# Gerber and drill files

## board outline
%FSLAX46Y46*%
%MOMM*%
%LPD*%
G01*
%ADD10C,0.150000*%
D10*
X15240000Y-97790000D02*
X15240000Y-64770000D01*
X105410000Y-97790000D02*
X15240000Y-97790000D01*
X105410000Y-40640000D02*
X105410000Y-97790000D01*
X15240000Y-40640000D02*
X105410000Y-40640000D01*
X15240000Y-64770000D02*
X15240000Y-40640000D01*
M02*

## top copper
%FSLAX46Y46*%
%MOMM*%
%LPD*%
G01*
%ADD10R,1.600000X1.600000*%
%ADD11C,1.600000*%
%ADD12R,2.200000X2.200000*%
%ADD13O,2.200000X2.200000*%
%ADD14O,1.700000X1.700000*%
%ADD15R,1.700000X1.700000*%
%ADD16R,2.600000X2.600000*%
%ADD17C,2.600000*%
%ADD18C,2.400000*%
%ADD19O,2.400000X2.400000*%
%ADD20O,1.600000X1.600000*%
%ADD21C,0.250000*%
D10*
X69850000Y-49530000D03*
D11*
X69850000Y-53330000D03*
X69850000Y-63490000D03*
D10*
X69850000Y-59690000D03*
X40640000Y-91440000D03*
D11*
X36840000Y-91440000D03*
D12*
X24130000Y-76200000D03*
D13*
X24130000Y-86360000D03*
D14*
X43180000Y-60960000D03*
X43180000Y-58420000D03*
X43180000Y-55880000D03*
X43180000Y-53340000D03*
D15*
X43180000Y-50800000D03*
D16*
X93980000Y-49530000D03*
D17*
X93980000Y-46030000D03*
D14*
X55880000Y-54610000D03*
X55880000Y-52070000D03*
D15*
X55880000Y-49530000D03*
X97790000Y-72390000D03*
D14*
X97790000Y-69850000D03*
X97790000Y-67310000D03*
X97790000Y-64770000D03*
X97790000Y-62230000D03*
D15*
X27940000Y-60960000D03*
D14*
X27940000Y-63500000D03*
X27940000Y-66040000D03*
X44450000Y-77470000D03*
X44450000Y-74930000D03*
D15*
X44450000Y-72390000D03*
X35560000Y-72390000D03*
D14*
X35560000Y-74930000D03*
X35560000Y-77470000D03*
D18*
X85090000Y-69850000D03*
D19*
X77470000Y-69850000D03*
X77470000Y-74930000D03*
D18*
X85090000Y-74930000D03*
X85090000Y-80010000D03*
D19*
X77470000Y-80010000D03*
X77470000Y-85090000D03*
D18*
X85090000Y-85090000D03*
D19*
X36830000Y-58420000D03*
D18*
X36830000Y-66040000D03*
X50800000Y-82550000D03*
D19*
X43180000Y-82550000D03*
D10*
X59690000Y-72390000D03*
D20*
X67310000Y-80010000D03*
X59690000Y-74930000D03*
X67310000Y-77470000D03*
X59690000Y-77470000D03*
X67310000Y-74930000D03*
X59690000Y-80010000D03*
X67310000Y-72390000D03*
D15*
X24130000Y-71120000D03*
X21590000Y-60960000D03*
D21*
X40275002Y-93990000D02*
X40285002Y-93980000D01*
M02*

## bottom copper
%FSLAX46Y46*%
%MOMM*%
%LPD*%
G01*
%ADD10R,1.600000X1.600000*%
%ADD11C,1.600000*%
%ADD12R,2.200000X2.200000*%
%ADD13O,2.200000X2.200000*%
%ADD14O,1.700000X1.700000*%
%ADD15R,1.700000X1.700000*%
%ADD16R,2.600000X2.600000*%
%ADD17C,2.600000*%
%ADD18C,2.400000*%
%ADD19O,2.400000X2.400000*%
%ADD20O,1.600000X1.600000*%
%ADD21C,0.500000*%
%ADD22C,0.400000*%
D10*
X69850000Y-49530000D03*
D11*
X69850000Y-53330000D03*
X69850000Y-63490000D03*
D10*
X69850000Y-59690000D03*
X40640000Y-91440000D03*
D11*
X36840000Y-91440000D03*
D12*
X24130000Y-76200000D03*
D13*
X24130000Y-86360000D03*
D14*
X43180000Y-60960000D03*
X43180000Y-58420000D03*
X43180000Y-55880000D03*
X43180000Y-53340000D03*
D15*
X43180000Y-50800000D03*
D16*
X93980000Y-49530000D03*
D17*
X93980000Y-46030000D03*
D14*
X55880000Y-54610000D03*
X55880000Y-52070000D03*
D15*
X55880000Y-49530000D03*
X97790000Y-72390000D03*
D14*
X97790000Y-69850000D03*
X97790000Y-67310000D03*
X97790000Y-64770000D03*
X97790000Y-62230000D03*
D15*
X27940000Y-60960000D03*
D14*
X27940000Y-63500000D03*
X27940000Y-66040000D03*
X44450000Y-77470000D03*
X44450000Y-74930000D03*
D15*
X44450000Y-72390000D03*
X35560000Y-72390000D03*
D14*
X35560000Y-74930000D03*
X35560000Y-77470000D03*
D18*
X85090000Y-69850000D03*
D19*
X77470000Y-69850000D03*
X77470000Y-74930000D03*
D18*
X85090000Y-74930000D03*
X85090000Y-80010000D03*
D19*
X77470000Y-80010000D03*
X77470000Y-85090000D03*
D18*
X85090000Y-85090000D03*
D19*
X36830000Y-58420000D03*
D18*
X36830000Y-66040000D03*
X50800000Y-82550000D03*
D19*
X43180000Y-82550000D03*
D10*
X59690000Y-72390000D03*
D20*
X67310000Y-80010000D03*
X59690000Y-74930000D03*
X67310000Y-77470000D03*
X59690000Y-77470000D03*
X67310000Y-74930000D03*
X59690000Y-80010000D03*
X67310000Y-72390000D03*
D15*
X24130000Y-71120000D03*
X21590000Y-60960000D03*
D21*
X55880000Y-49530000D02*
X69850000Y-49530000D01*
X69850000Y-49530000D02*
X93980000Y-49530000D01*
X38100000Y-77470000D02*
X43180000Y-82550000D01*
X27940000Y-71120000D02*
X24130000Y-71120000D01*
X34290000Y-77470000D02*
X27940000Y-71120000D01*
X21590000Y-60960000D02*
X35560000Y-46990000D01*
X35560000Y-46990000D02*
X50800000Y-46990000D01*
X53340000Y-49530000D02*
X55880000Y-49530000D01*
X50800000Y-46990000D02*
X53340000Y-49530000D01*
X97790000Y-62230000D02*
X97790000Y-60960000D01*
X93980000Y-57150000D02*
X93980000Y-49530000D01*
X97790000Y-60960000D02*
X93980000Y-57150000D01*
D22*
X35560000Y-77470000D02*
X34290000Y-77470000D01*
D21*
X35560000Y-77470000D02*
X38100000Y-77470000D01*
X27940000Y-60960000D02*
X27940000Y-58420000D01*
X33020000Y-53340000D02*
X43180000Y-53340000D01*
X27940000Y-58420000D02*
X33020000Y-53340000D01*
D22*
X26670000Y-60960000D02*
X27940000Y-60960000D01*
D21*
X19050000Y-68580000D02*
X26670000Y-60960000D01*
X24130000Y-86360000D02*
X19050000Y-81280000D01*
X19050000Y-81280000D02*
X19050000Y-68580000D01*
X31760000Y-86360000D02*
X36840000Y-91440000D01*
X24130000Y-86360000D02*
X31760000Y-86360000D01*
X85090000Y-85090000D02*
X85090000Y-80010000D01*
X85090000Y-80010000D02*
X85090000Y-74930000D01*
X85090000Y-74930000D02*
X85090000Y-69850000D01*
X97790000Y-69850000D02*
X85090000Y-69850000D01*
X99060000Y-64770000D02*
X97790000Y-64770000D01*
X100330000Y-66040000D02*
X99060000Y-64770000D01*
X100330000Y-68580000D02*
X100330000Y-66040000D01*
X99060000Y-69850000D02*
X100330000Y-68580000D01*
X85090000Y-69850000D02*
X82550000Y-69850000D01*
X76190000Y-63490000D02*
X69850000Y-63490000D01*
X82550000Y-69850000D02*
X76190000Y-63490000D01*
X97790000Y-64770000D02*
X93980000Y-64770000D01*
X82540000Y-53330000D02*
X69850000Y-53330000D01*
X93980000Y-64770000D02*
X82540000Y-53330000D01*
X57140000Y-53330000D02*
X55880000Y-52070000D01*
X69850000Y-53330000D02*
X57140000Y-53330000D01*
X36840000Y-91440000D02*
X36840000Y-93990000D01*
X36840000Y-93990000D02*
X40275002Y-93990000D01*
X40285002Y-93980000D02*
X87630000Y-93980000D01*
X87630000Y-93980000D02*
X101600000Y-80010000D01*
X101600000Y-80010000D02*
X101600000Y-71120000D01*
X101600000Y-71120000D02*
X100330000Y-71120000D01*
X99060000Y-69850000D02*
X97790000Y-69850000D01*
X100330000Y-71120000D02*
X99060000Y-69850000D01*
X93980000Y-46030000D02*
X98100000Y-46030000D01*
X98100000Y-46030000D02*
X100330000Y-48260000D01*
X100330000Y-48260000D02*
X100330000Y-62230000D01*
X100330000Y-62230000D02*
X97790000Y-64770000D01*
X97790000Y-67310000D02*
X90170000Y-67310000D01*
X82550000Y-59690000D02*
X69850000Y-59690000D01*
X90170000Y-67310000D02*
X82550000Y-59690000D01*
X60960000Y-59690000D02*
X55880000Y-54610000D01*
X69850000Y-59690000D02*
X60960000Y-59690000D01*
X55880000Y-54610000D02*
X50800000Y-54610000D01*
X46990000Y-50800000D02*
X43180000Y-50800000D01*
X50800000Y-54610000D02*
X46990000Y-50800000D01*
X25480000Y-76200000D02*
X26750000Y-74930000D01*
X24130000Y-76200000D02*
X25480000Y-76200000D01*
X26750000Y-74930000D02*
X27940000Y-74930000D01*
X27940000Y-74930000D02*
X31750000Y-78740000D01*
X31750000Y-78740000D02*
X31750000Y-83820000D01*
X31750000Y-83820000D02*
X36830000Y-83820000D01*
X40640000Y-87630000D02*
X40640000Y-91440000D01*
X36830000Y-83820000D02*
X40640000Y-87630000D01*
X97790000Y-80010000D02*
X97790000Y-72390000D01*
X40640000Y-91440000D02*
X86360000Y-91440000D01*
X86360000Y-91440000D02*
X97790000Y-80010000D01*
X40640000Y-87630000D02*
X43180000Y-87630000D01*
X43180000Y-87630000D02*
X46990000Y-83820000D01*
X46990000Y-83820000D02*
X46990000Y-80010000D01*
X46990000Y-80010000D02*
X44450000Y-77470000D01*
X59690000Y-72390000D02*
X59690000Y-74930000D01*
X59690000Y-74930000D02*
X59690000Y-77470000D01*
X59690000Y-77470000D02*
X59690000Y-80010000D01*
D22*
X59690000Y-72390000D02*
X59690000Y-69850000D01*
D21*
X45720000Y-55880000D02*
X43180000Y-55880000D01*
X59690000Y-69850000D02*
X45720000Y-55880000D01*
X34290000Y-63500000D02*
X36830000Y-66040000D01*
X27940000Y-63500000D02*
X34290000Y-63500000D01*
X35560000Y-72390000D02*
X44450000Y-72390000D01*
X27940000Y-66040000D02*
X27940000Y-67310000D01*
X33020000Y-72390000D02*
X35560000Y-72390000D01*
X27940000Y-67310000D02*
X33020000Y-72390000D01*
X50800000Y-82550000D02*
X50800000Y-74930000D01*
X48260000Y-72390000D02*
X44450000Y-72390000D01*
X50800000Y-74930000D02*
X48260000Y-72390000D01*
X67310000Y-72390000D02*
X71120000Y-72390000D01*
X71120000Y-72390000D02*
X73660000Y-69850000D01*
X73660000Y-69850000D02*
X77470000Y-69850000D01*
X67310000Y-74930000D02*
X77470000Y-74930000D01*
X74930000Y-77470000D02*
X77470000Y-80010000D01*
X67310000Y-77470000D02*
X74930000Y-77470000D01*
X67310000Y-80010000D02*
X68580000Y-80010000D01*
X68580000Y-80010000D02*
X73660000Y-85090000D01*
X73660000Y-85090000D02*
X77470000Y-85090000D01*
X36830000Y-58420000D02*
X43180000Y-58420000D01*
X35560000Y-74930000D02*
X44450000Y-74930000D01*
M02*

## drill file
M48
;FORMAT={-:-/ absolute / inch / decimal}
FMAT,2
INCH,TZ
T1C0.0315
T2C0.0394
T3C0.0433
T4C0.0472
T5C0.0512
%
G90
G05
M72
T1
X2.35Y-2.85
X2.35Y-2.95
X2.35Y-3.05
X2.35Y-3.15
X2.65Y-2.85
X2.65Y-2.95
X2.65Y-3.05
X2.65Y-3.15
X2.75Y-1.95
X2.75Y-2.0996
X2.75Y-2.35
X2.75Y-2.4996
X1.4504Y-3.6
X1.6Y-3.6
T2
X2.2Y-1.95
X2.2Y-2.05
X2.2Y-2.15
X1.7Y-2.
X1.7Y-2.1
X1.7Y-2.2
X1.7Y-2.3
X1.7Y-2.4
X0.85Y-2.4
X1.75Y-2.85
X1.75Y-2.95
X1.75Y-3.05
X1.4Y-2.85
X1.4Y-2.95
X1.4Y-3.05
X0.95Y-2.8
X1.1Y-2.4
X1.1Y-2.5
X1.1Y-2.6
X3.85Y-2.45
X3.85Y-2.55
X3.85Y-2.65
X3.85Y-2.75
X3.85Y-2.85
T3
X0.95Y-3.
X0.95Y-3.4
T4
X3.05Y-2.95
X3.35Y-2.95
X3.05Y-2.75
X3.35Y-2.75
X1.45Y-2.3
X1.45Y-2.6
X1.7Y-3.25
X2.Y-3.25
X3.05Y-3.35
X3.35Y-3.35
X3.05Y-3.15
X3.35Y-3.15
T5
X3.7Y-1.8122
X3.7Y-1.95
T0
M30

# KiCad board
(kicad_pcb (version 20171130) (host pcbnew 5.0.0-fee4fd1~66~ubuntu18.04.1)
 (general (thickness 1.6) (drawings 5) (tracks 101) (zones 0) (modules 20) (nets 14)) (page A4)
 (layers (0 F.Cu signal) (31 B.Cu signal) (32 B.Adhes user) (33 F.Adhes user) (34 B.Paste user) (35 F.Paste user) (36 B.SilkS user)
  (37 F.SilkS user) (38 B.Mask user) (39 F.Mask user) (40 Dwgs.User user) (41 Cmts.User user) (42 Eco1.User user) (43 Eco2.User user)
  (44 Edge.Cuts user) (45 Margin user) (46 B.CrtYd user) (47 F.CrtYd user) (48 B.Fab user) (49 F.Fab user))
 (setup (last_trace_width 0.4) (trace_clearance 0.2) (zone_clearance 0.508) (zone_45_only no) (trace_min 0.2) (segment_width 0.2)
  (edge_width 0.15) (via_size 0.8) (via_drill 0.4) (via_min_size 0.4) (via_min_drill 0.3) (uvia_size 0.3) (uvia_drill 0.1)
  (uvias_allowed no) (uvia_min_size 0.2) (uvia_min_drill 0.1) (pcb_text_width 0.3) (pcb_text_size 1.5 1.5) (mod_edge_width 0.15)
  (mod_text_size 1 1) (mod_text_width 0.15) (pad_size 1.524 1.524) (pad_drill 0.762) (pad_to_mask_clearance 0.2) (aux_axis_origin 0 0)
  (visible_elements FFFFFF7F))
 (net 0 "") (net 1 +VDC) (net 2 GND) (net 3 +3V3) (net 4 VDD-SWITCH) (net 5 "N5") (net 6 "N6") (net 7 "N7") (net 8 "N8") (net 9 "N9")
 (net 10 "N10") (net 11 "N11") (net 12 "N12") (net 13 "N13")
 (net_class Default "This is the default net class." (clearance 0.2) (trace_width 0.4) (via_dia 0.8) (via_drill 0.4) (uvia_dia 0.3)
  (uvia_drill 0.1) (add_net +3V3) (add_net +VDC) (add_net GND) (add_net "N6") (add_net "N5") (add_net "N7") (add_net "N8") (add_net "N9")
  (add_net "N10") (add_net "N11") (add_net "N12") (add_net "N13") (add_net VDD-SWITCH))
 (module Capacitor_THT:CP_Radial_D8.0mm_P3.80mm (layer F.Cu) (at 69.85 49.53 270)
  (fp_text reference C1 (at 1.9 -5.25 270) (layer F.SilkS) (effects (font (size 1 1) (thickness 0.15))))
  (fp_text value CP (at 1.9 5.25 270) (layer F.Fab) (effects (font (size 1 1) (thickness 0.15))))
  (pad 1 thru_hole rect (at 0 0 270) (size 1.6 1.6) (drill 0.8) (layers *.Cu *.Mask) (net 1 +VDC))
  (pad 2 thru_hole circle (at 3.8 0 270) (size 1.6 1.6) (drill 0.8) (layers *.Cu *.Mask) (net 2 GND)))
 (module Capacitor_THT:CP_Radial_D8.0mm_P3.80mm (layer F.Cu) (at 69.85 59.69 270)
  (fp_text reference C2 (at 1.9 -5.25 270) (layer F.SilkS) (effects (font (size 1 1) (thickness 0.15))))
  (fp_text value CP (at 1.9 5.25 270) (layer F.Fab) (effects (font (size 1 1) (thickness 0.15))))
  (pad 2 thru_hole circle (at 3.8 0 270) (size 1.6 1.6) (drill 0.8) (layers *.Cu *.Mask) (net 2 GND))
  (pad 1 thru_hole rect (at 0 0 270) (size 1.6 1.6) (drill 0.8) (layers *.Cu *.Mask) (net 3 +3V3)))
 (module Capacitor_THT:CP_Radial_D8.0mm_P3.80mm (layer F.Cu) (at 40.64 91.44 180)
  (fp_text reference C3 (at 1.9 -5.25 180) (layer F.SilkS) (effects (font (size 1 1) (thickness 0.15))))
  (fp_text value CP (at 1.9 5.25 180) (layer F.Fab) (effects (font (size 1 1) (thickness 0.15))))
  (pad 1 thru_hole rect (at 0 0 180) (size 1.6 1.6) (drill 0.8) (layers *.Cu *.Mask) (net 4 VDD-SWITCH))
  (pad 2 thru_hole circle (at 3.8 0 180) (size 1.6 1.6) (drill 0.8) (layers *.Cu *.Mask) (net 2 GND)))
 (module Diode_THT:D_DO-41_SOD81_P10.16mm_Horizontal (layer F.Cu) (at 24.13 76.2 270)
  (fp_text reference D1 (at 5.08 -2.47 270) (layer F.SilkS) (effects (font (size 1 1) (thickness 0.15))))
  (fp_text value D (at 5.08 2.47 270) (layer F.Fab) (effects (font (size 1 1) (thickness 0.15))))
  (pad 1 thru_hole rect (at 0 0 270) (size 2.2 2.2) (drill 1.1) (layers *.Cu *.Mask) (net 4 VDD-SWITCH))
  (pad 2 thru_hole oval (at 10.16 0 270) (size 2.2 2.2) (drill 1.1) (layers *.Cu *.Mask) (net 2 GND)))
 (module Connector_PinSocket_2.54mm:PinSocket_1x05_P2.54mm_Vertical (layer F.Cu) (at 43.18 50.8)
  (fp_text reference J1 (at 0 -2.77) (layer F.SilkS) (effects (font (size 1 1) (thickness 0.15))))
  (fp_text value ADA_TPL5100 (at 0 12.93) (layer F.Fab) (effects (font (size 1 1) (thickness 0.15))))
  (pad 5 thru_hole oval (at 0 10.16) (size 1.7 1.7) (drill 1) (layers *.Cu *.Mask))
  (pad 4 thru_hole oval (at 0 7.62) (size 1.7 1.7) (drill 1) (layers *.Cu *.Mask) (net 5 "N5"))
  (pad 3 thru_hole oval (at 0 5.08) (size 1.7 1.7) (drill 1) (layers *.Cu *.Mask) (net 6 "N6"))
  (pad 2 thru_hole oval (at 0 2.54) (size 1.7 1.7) (drill 1) (layers *.Cu *.Mask) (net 2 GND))
  (pad 1 thru_hole rect (at 0 0) (size 1.7 1.7) (drill 1) (layers *.Cu *.Mask) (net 3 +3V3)))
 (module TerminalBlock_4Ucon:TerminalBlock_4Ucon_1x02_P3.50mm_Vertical (layer F.Cu) (at 93.98 49.53 90)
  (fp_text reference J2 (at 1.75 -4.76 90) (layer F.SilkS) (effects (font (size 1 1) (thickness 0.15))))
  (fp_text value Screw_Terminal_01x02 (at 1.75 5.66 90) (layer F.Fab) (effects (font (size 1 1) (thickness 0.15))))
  (pad 1 thru_hole rect (at 0 0 90) (size 2.6 2.6) (drill 1.3) (layers *.Cu *.Mask) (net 1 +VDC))
  (pad 2 thru_hole circle (at 3.5 0 90) (size 2.6 2.6) (drill 1.3) (layers *.Cu *.Mask) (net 2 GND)))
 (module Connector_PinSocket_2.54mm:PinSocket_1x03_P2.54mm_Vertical (layer F.Cu) (at 55.88 49.53)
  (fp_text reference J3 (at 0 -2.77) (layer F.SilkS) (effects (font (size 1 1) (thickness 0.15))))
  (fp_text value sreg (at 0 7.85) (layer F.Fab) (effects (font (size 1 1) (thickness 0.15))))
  (pad 3 thru_hole oval (at 0 5.08) (size 1.7 1.7) (drill 1) (layers *.Cu *.Mask) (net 3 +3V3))
  (pad 2 thru_hole oval (at 0 2.54) (size 1.7 1.7) (drill 1) (layers *.Cu *.Mask) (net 2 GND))
  (pad 1 thru_hole rect (at 0 0) (size 1.7 1.7) (drill 1) (layers *.Cu *.Mask) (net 1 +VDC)))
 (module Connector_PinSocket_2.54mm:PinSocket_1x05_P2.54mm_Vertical (layer F.Cu) (at 97.79 72.39 180)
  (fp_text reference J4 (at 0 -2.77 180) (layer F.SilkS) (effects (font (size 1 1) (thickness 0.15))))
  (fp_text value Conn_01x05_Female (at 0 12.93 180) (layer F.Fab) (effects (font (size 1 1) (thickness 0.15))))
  (pad 1 thru_hole rect (at 0 0 180) (size 1.7 1.7) (drill 1) (layers *.Cu *.Mask) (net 4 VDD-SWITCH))
  (pad 2 thru_hole oval (at 0 2.54 180) (size 1.7 1.7) (drill 1) (layers *.Cu *.Mask) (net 2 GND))
  (pad 3 thru_hole oval (at 0 5.08 180) (size 1.7 1.7) (drill 1) (layers *.Cu *.Mask) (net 3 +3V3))
  (pad 4 thru_hole oval (at 0 7.62 180) (size 1.7 1.7) (drill 1) (layers *.Cu *.Mask) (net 2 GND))
  (pad 5 thru_hole oval (at 0 10.16 180) (size 1.7 1.7) (drill 1) (layers *.Cu *.Mask) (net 1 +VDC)))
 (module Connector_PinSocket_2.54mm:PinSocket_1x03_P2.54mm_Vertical (layer F.Cu) (at 27.94 60.96)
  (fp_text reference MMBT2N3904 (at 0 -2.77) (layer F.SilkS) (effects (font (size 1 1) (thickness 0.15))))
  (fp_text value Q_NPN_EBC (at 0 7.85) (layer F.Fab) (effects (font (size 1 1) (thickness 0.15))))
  (pad 1 thru_hole rect (at 0 0) (size 1.7 1.7) (drill 1) (layers *.Cu *.Mask) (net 2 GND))
  (pad 2 thru_hole oval (at 0 2.54) (size 1.7 1.7) (drill 1) (layers *.Cu *.Mask) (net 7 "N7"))
  (pad 3 thru_hole oval (at 0 5.08) (size 1.7 1.7) (drill 1) (layers *.Cu *.Mask) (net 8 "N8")))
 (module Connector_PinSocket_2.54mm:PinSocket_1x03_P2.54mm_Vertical (layer F.Cu) (at 44.45 72.39)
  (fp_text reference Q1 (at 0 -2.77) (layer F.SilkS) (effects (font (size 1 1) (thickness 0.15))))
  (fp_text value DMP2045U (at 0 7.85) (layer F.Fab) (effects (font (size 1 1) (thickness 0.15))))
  (pad 3 thru_hole oval (at 0 5.08) (size 1.7 1.7) (drill 1) (layers *.Cu *.Mask) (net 4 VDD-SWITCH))
  (pad 2 thru_hole oval (at 0 2.54) (size 1.7 1.7) (drill 1) (layers *.Cu *.Mask) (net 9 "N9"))
  (pad 1 thru_hole rect (at 0 0) (size 1.7 1.7) (drill 1) (layers *.Cu *.Mask) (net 8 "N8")))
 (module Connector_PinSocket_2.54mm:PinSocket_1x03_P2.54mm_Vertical (layer F.Cu) (at 35.56 72.39)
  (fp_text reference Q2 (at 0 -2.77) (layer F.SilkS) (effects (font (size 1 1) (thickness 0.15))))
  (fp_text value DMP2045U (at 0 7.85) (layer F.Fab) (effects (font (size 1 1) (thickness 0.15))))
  (pad 1 thru_hole rect (at 0 0) (size 1.7 1.7) (drill 1) (layers *.Cu *.Mask) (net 8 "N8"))
  (pad 2 thru_hole oval (at 0 2.54) (size 1.7 1.7) (drill 1) (layers *.Cu *.Mask) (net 9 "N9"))
  (pad 3 thru_hole oval (at 0 5.08) (size 1.7 1.7) (drill 1) (layers *.Cu *.Mask) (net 1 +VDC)))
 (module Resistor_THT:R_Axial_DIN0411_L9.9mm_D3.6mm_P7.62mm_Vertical (layer F.Cu) (at 85.09 69.85 180)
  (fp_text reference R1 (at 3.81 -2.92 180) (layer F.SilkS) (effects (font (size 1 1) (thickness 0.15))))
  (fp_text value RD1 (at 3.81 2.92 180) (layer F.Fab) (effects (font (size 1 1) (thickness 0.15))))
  (pad 1 thru_hole circle (at 0 0 180) (size 2.4 2.4) (drill 1.2) (layers *.Cu *.Mask) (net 2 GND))
  (pad 2 thru_hole oval (at 7.62 0 180) (size 2.4 2.4) (drill 1.2) (layers *.Cu *.Mask) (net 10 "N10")))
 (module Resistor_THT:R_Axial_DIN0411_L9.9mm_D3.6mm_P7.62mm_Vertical (layer F.Cu) (at 85.09 74.93 180)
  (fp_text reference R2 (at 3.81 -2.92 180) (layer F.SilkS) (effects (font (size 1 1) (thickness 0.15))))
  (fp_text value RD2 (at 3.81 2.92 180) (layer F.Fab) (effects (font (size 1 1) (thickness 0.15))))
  (pad 2 thru_hole oval (at 7.62 0 180) (size 2.4 2.4) (drill 1.2) (layers *.Cu *.Mask) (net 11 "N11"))
  (pad 1 thru_hole circle (at 0 0 180) (size 2.4 2.4) (drill 1.2) (layers *.Cu *.Mask) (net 2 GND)))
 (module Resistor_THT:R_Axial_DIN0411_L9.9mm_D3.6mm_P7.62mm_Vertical (layer F.Cu) (at 85.09 80.01 180)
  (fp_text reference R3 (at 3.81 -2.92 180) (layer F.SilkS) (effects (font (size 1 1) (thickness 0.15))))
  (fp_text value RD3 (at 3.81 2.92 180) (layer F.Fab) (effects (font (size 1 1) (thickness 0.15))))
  (pad 1 thru_hole circle (at 0 0 180) (size 2.4 2.4) (drill 1.2) (layers *.Cu *.Mask) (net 2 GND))
  (pad 2 thru_hole oval (at 7.62 0 180) (size 2.4 2.4) (drill 1.2) (layers *.Cu *.Mask) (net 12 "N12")))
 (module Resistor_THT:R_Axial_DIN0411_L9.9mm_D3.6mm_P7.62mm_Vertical (layer F.Cu) (at 85.09 85.09 180)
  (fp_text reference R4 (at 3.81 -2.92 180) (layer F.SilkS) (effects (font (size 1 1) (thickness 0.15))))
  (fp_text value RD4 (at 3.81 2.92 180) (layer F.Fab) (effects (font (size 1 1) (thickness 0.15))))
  (pad 2 thru_hole oval (at 7.62 0 180) (size 2.4 2.4) (drill 1.2) (layers *.Cu *.Mask) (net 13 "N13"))
  (pad 1 thru_hole circle (at 0 0 180) (size 2.4 2.4) (drill 1.2) (layers *.Cu *.Mask) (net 2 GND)))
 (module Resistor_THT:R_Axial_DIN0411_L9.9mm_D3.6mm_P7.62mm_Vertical (layer F.Cu) (at 36.83 66.04 90)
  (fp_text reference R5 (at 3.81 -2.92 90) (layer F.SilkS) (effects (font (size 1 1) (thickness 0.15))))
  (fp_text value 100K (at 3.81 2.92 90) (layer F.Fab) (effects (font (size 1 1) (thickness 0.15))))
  (pad 2 thru_hole oval (at 7.62 0 90) (size 2.4 2.4) (drill 1.2) (layers *.Cu *.Mask) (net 5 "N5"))
  (pad 1 thru_hole circle (at 0 0 90) (size 2.4 2.4) (drill 1.2) (layers *.Cu *.Mask) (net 7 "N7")))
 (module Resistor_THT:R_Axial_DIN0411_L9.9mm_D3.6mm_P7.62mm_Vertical (layer F.Cu) (at 50.8 82.55 180)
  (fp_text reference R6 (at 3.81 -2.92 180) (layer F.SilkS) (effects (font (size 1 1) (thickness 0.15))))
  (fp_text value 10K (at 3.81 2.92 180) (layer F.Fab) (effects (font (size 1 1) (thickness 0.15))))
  (pad 1 thru_hole circle (at 0 0 180) (size 2.4 2.4) (drill 1.2) (layers *.Cu *.Mask) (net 8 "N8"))
  (pad 2 thru_hole oval (at 7.62 0 180) (size 2.4 2.4) (drill 1.2) (layers *.Cu *.Mask) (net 1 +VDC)))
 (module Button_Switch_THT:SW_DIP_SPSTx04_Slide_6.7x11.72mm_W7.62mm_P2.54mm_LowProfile (layer F.Cu) (at 59.69 72.39)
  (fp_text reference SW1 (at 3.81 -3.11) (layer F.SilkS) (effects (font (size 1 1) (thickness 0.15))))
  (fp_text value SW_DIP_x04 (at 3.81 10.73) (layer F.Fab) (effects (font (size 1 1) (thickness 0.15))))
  (pad 1 thru_hole rect (at 0 0) (size 1.6 1.6) (drill 0.8) (layers *.Cu *.Mask) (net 6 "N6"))
  (pad 5 thru_hole oval (at 7.62 7.62) (size 1.6 1.6) (drill 0.8) (layers *.Cu *.Mask) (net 13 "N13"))
  (pad 2 thru_hole oval (at 0 2.54) (size 1.6 1.6) (drill 0.8) (layers *.Cu *.Mask) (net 6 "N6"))
  (pad 6 thru_hole oval (at 7.62 5.08) (size 1.6 1.6) (drill 0.8) (layers *.Cu *.Mask) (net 12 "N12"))
  (pad 3 thru_hole oval (at 0 5.08) (size 1.6 1.6) (drill 0.8) (layers *.Cu *.Mask) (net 6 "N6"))
  (pad 7 thru_hole oval (at 7.62 2.54) (size 1.6 1.6) (drill 0.8) (layers *.Cu *.Mask) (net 11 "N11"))
  (pad 4 thru_hole oval (at 0 7.62) (size 1.6 1.6) (drill 0.8) (layers *.Cu *.Mask) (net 6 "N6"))
  (pad 8 thru_hole oval (at 7.62 0) (size 1.6 1.6) (drill 0.8) (layers *.Cu *.Mask) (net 10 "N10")))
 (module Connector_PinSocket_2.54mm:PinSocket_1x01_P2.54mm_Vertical (layer F.Cu) (at 24.13 71.12)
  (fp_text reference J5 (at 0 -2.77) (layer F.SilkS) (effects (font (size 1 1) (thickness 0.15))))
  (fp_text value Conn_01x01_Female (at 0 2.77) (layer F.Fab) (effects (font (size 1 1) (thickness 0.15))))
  (pad 1 thru_hole rect (at 0 0) (size 1.7 1.7) (drill 1) (layers *.Cu *.Mask) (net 1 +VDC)))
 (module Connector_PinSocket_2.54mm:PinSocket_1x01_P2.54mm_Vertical (layer F.Cu) (at 21.59 60.96)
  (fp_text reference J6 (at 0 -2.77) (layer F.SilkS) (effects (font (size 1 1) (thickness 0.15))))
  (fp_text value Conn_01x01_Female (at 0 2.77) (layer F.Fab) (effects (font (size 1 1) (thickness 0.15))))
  (pad 1 thru_hole rect (at 0 0) (size 1.7 1.7) (drill 1) (layers *.Cu *.Mask) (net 1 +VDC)))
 (gr_line (start 15.24 97.79) (end 15.24 64.77) (layer Edge.Cuts) (width 0.15))
 (gr_line (start 105.41 97.79) (end 15.24 97.79) (layer Edge.Cuts) (width 0.15))
 (gr_line (start 105.41 40.64) (end 105.41 97.79) (layer Edge.Cuts) (width 0.15))
 (gr_line (start 15.24 40.64) (end 105.41 40.64) (layer Edge.Cuts) (width 0.15))
 (gr_line (start 15.24 64.77) (end 15.24 40.64) (layer Edge.Cuts) (width 0.15))
 (segment (start 55.88 49.53) (end 69.85 49.53) (width 0.5) (layer B.Cu) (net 1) (status 30))
 (segment (start 69.85 49.53) (end 93.98 49.53) (width 0.5) (layer B.Cu) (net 1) (status 30))
 (segment (start 38.1 77.47) (end 43.18 82.55) (width 0.5) (layer B.Cu) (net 1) (status 20))
 (segment (start 27.94 71.12) (end 24.13 71.12) (width 0.5) (layer B.Cu) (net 1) (status 20))
 (segment (start 34.29 77.47) (end 27.94 71.12) (width 0.5) (layer B.Cu) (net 1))
 (segment (start 21.59 60.96) (end 35.56 46.99) (width 0.5) (layer B.Cu) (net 1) (status 10))
 (segment (start 35.56 46.99) (end 50.8 46.99) (width 0.5) (layer B.Cu) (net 1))
 (segment (start 53.34 49.53) (end 55.88 49.53) (width 0.5) (layer B.Cu) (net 1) (status 20))
 (segment (start 50.8 46.99) (end 53.34 49.53) (width 0.5) (layer B.Cu) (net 1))
 (segment (start 97.79 62.23) (end 97.79 60.96) (width 0.5) (layer B.Cu) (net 1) (status 10))
 (segment (start 93.98 57.15) (end 93.98 49.53) (width 0.5) (layer B.Cu) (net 1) (status 20))
 (segment (start 97.79 60.96) (end 93.98 57.15) (width 0.5) (layer B.Cu) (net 1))
 (segment (start 35.56 77.47) (end 34.29 77.47) (width 0.4) (layer B.Cu) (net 1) (status 10))
 (segment (start 35.56 77.47) (end 38.1 77.47) (width 0.5) (layer B.Cu) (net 1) (status 10))
 (segment (start 27.94 60.96) (end 27.94 58.42) (width 0.5) (layer B.Cu) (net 2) (status 10))
 (segment (start 33.02 53.34) (end 43.18 53.34) (width 0.5) (layer B.Cu) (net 2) (status 20))
 (segment (start 27.94 58.42) (end 33.02 53.34) (width 0.5) (layer B.Cu) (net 2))
 (segment (start 26.67 60.96) (end 27.94 60.96) (width 0.4) (layer B.Cu) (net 2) (status 20))
 (segment (start 19.05 68.58) (end 26.67 60.96) (width 0.5) (layer B.Cu) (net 2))
 (segment (start 24.13 86.36) (end 19.05 81.28) (width 0.5) (layer B.Cu) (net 2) (status 10))
 (segment (start 19.05 81.28) (end 19.05 68.58) (width 0.5) (layer B.Cu) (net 2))
 (segment (start 31.76 86.36) (end 36.84 91.44) (width 0.5) (layer B.Cu) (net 2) (status 20))
 (segment (start 24.13 86.36) (end 31.76 86.36) (width 0.5) (layer B.Cu) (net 2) (status 10))
 (segment (start 85.09 85.09) (end 85.09 80.01) (width 0.5) (layer B.Cu) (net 2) (status 30))
 (segment (start 85.09 80.01) (end 85.09 74.93) (width 0.5) (layer B.Cu) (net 2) (status 30))
 (segment (start 85.09 74.93) (end 85.09 69.85) (width 0.5) (layer B.Cu) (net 2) (status 30))
 (segment (start 97.79 69.85) (end 85.09 69.85) (width 0.5) (layer B.Cu) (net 2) (status 30))
 (segment (start 99.06 64.77) (end 97.79 64.77) (width 0.5) (layer B.Cu) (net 2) (status 20))
 (segment (start 100.33 66.04) (end 99.06 64.77) (width 0.5) (layer B.Cu) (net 2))
 (segment (start 100.33 68.58) (end 100.33 66.04) (width 0.5) (layer B.Cu) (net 2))
 (segment (start 99.06 69.85) (end 100.33 68.58) (width 0.5) (layer B.Cu) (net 2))
 (segment (start 85.09 69.85) (end 82.55 69.85) (width 0.5) (layer B.Cu) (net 2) (status 10))
 (segment (start 76.19 63.49) (end 69.85 63.49) (width 0.5) (layer B.Cu) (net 2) (status 20))
 (segment (start 82.55 69.85) (end 76.19 63.49) (width 0.5) (layer B.Cu) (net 2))
 (segment (start 97.79 64.77) (end 93.98 64.77) (width 0.5) (layer B.Cu) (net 2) (status 10))
 (segment (start 82.54 53.33) (end 69.85 53.33) (width 0.5) (layer B.Cu) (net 2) (status 20))
 (segment (start 93.98 64.77) (end 82.54 53.33) (width 0.5) (layer B.Cu) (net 2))
 (segment (start 57.14 53.33) (end 55.88 52.07) (width 0.5) (layer B.Cu) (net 2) (status 20))
 (segment (start 69.85 53.33) (end 57.14 53.33) (width 0.5) (layer B.Cu) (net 2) (status 10))
 (segment (start 36.84 91.44) (end 36.84 93.99) (width 0.5) (layer B.Cu) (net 2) (status 10))
 (segment (start 40.275002 93.99) (end 40.285002 93.98) (width 0.25) (layer F.Cu) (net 2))
 (segment (start 36.84 93.99) (end 40.275002 93.99) (width 0.5) (layer B.Cu) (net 2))
 (segment (start 40.285002 93.98) (end 87.63 93.98) (width 0.5) (layer B.Cu) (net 2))
 (segment (start 87.63 93.98) (end 101.6 80.01) (width 0.5) (layer B.Cu) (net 2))
 (segment (start 101.6 80.01) (end 101.6 71.12) (width 0.5) (layer B.Cu) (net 2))
 (segment (start 101.6 71.12) (end 100.33 71.12) (width 0.5) (layer B.Cu) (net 2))
 (segment (start 99.06 69.85) (end 97.79 69.85) (width 0.5) (layer B.Cu) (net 2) (status 20))
 (segment (start 100.33 71.12) (end 99.06 69.85) (width 0.5) (layer B.Cu) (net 2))
 (segment (start 93.98 46.03) (end 98.1 46.03) (width 0.5) (layer B.Cu) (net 2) (status 10))
 (segment (start 98.1 46.03) (end 100.33 48.26) (width 0.5) (layer B.Cu) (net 2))
 (segment (start 100.33 48.26) (end 100.33 62.23) (width 0.5) (layer B.Cu) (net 2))
 (segment (start 100.33 62.23) (end 97.79 64.77) (width 0.5) (layer B.Cu) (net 2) (status 20))
 (segment (start 97.79 67.31) (end 90.17 67.31) (width 0.5) (layer B.Cu) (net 3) (status 10))
 (segment (start 82.55 59.69) (end 69.85 59.69) (width 0.5) (layer B.Cu) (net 3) (status 20))
 (segment (start 90.17 67.31) (end 82.55 59.69) (width 0.5) (layer B.Cu) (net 3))
 (segment (start 60.96 59.69) (end 55.88 54.61) (width 0.5) (layer B.Cu) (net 3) (status 20))
 (segment (start 69.85 59.69) (end 60.96 59.69) (width 0.5) (layer B.Cu) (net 3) (status 10))
 (segment (start 55.88 54.61) (end 50.8 54.61) (width 0.5) (layer B.Cu) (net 3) (status 10))
 (segment (start 46.99 50.8) (end 43.18 50.8) (width 0.5) (layer B.Cu) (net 3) (status 20))
 (segment (start 50.8 54.61) (end 46.99 50.8) (width 0.5) (layer B.Cu) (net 3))
 (segment (start 25.48 76.2) (end 26.75 74.93) (width 0.5) (layer B.Cu) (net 4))
 (segment (start 24.13 76.2) (end 25.48 76.2) (width 0.5) (layer B.Cu) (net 4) (status 10))
 (segment (start 26.75 74.93) (end 27.94 74.93) (width 0.5) (layer B.Cu) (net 4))
 (segment (start 27.94 74.93) (end 31.75 78.74) (width 0.5) (layer B.Cu) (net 4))
 (segment (start 31.75 78.74) (end 31.75 83.82) (width 0.5) (layer B.Cu) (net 4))
 (segment (start 31.75 83.82) (end 36.83 83.82) (width 0.5) (layer B.Cu) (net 4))
 (segment (start 40.64 87.63) (end 40.64 91.44) (width 0.5) (layer B.Cu) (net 4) (status 20))
 (segment (start 36.83 83.82) (end 40.64 87.63) (width 0.5) (layer B.Cu) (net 4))
 (segment (start 97.79 80.01) (end 97.79 72.39) (width 0.5) (layer B.Cu) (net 4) (status 20))
 (segment (start 40.64 91.44) (end 86.36 91.44) (width 0.5) (layer B.Cu) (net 4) (status 10))
 (segment (start 86.36 91.44) (end 97.79 80.01) (width 0.5) (layer B.Cu) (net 4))
 (segment (start 40.64 87.63) (end 43.18 87.63) (width 0.5) (layer B.Cu) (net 4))
 (segment (start 43.18 87.63) (end 46.99 83.82) (width 0.5) (layer B.Cu) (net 4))
 (segment (start 46.99 83.82) (end 46.99 80.01) (width 0.5) (layer B.Cu) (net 4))
 (segment (start 46.99 80.01) (end 44.45 77.47) (width 0.5) (layer B.Cu) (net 4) (status 20))
 (segment (start 59.69 72.39) (end 59.69 74.93) (width 0.5) (layer B.Cu) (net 6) (status 30))
 (segment (start 59.69 74.93) (end 59.69 77.47) (width 0.5) (layer B.Cu) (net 6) (status 30))
 (segment (start 59.69 77.47) (end 59.69 80.01) (width 0.5) (layer B.Cu) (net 6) (status 30))
 (segment (start 59.69 69.85) (end 45.72 55.88) (width 0.5) (layer B.Cu) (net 6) (status 1000000))
 (segment (start 45.72 55.88) (end 43.18 55.88) (width 0.5) (layer B.Cu) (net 6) (status 1000020))
 (segment (start 59.69 72.39) (end 59.69 69.85) (width 0.4) (layer B.Cu) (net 6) (status 1000010))
 (segment (start 34.29 63.5) (end 36.83 66.04) (width 0.5) (layer B.Cu) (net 7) (status 20))
 (segment (start 27.94 63.5) (end 34.29 63.5) (width 0.5) (layer B.Cu) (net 7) (status 10))
 (segment (start 35.56 72.39) (end 44.45 72.39) (width 0.5) (layer B.Cu) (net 8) (status 30))
 (segment (start 27.94 66.04) (end 27.94 67.31) (width 0.5) (layer B.Cu) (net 8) (status 10))
 (segment (start 33.02 72.39) (end 35.56 72.39) (width 0.5) (layer B.Cu) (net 8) (status 20))
 (segment (start 27.94 67.31) (end 33.02 72.39) (width 0.5) (layer B.Cu) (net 8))
 (segment (start 50.8 82.55) (end 50.8 74.93) (width 0.5) (layer B.Cu) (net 8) (status 10))
 (segment (start 48.26 72.39) (end 44.45 72.39) (width 0.5) (layer B.Cu) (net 8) (status 20))
 (segment (start 50.8 74.93) (end 48.26 72.39) (width 0.5) (layer B.Cu) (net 8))
 (segment (start 67.31 72.39) (end 71.12 72.39) (width 0.5) (layer B.Cu) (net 10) (status 10))
 (segment (start 71.12 72.39) (end 73.66 69.85) (width 0.5) (layer B.Cu) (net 10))
 (segment (start 73.66 69.85) (end 77.47 69.85) (width 0.5) (layer B.Cu) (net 10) (status 20))
 (segment (start 67.31 74.93) (end 77.47 74.93) (width 0.5) (layer B.Cu) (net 11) (status 30))
 (segment (start 74.93 77.47) (end 77.47 80.01) (width 0.5) (layer B.Cu) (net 12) (status 20))
 (segment (start 67.31 77.47) (end 74.93 77.47) (width 0.5) (layer B.Cu) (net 12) (status 10))
 (segment (start 67.31 80.01) (end 68.58 80.01) (width 0.5) (layer B.Cu) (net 13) (status 10))
 (segment (start 68.58 80.01) (end 73.66 85.09) (width 0.5) (layer B.Cu) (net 13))
 (segment (start 73.66 85.09) (end 77.47 85.09) (width 0.5) (layer B.Cu) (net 13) (status 20))
 (segment (start 36.83 58.42) (end 43.18 58.42) (width 0.5) (layer B.Cu) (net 5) (status 30))
 (segment (start 35.56 74.93) (end 44.45 74.93) (width 0.5) (layer B.Cu) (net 9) (status 30)))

